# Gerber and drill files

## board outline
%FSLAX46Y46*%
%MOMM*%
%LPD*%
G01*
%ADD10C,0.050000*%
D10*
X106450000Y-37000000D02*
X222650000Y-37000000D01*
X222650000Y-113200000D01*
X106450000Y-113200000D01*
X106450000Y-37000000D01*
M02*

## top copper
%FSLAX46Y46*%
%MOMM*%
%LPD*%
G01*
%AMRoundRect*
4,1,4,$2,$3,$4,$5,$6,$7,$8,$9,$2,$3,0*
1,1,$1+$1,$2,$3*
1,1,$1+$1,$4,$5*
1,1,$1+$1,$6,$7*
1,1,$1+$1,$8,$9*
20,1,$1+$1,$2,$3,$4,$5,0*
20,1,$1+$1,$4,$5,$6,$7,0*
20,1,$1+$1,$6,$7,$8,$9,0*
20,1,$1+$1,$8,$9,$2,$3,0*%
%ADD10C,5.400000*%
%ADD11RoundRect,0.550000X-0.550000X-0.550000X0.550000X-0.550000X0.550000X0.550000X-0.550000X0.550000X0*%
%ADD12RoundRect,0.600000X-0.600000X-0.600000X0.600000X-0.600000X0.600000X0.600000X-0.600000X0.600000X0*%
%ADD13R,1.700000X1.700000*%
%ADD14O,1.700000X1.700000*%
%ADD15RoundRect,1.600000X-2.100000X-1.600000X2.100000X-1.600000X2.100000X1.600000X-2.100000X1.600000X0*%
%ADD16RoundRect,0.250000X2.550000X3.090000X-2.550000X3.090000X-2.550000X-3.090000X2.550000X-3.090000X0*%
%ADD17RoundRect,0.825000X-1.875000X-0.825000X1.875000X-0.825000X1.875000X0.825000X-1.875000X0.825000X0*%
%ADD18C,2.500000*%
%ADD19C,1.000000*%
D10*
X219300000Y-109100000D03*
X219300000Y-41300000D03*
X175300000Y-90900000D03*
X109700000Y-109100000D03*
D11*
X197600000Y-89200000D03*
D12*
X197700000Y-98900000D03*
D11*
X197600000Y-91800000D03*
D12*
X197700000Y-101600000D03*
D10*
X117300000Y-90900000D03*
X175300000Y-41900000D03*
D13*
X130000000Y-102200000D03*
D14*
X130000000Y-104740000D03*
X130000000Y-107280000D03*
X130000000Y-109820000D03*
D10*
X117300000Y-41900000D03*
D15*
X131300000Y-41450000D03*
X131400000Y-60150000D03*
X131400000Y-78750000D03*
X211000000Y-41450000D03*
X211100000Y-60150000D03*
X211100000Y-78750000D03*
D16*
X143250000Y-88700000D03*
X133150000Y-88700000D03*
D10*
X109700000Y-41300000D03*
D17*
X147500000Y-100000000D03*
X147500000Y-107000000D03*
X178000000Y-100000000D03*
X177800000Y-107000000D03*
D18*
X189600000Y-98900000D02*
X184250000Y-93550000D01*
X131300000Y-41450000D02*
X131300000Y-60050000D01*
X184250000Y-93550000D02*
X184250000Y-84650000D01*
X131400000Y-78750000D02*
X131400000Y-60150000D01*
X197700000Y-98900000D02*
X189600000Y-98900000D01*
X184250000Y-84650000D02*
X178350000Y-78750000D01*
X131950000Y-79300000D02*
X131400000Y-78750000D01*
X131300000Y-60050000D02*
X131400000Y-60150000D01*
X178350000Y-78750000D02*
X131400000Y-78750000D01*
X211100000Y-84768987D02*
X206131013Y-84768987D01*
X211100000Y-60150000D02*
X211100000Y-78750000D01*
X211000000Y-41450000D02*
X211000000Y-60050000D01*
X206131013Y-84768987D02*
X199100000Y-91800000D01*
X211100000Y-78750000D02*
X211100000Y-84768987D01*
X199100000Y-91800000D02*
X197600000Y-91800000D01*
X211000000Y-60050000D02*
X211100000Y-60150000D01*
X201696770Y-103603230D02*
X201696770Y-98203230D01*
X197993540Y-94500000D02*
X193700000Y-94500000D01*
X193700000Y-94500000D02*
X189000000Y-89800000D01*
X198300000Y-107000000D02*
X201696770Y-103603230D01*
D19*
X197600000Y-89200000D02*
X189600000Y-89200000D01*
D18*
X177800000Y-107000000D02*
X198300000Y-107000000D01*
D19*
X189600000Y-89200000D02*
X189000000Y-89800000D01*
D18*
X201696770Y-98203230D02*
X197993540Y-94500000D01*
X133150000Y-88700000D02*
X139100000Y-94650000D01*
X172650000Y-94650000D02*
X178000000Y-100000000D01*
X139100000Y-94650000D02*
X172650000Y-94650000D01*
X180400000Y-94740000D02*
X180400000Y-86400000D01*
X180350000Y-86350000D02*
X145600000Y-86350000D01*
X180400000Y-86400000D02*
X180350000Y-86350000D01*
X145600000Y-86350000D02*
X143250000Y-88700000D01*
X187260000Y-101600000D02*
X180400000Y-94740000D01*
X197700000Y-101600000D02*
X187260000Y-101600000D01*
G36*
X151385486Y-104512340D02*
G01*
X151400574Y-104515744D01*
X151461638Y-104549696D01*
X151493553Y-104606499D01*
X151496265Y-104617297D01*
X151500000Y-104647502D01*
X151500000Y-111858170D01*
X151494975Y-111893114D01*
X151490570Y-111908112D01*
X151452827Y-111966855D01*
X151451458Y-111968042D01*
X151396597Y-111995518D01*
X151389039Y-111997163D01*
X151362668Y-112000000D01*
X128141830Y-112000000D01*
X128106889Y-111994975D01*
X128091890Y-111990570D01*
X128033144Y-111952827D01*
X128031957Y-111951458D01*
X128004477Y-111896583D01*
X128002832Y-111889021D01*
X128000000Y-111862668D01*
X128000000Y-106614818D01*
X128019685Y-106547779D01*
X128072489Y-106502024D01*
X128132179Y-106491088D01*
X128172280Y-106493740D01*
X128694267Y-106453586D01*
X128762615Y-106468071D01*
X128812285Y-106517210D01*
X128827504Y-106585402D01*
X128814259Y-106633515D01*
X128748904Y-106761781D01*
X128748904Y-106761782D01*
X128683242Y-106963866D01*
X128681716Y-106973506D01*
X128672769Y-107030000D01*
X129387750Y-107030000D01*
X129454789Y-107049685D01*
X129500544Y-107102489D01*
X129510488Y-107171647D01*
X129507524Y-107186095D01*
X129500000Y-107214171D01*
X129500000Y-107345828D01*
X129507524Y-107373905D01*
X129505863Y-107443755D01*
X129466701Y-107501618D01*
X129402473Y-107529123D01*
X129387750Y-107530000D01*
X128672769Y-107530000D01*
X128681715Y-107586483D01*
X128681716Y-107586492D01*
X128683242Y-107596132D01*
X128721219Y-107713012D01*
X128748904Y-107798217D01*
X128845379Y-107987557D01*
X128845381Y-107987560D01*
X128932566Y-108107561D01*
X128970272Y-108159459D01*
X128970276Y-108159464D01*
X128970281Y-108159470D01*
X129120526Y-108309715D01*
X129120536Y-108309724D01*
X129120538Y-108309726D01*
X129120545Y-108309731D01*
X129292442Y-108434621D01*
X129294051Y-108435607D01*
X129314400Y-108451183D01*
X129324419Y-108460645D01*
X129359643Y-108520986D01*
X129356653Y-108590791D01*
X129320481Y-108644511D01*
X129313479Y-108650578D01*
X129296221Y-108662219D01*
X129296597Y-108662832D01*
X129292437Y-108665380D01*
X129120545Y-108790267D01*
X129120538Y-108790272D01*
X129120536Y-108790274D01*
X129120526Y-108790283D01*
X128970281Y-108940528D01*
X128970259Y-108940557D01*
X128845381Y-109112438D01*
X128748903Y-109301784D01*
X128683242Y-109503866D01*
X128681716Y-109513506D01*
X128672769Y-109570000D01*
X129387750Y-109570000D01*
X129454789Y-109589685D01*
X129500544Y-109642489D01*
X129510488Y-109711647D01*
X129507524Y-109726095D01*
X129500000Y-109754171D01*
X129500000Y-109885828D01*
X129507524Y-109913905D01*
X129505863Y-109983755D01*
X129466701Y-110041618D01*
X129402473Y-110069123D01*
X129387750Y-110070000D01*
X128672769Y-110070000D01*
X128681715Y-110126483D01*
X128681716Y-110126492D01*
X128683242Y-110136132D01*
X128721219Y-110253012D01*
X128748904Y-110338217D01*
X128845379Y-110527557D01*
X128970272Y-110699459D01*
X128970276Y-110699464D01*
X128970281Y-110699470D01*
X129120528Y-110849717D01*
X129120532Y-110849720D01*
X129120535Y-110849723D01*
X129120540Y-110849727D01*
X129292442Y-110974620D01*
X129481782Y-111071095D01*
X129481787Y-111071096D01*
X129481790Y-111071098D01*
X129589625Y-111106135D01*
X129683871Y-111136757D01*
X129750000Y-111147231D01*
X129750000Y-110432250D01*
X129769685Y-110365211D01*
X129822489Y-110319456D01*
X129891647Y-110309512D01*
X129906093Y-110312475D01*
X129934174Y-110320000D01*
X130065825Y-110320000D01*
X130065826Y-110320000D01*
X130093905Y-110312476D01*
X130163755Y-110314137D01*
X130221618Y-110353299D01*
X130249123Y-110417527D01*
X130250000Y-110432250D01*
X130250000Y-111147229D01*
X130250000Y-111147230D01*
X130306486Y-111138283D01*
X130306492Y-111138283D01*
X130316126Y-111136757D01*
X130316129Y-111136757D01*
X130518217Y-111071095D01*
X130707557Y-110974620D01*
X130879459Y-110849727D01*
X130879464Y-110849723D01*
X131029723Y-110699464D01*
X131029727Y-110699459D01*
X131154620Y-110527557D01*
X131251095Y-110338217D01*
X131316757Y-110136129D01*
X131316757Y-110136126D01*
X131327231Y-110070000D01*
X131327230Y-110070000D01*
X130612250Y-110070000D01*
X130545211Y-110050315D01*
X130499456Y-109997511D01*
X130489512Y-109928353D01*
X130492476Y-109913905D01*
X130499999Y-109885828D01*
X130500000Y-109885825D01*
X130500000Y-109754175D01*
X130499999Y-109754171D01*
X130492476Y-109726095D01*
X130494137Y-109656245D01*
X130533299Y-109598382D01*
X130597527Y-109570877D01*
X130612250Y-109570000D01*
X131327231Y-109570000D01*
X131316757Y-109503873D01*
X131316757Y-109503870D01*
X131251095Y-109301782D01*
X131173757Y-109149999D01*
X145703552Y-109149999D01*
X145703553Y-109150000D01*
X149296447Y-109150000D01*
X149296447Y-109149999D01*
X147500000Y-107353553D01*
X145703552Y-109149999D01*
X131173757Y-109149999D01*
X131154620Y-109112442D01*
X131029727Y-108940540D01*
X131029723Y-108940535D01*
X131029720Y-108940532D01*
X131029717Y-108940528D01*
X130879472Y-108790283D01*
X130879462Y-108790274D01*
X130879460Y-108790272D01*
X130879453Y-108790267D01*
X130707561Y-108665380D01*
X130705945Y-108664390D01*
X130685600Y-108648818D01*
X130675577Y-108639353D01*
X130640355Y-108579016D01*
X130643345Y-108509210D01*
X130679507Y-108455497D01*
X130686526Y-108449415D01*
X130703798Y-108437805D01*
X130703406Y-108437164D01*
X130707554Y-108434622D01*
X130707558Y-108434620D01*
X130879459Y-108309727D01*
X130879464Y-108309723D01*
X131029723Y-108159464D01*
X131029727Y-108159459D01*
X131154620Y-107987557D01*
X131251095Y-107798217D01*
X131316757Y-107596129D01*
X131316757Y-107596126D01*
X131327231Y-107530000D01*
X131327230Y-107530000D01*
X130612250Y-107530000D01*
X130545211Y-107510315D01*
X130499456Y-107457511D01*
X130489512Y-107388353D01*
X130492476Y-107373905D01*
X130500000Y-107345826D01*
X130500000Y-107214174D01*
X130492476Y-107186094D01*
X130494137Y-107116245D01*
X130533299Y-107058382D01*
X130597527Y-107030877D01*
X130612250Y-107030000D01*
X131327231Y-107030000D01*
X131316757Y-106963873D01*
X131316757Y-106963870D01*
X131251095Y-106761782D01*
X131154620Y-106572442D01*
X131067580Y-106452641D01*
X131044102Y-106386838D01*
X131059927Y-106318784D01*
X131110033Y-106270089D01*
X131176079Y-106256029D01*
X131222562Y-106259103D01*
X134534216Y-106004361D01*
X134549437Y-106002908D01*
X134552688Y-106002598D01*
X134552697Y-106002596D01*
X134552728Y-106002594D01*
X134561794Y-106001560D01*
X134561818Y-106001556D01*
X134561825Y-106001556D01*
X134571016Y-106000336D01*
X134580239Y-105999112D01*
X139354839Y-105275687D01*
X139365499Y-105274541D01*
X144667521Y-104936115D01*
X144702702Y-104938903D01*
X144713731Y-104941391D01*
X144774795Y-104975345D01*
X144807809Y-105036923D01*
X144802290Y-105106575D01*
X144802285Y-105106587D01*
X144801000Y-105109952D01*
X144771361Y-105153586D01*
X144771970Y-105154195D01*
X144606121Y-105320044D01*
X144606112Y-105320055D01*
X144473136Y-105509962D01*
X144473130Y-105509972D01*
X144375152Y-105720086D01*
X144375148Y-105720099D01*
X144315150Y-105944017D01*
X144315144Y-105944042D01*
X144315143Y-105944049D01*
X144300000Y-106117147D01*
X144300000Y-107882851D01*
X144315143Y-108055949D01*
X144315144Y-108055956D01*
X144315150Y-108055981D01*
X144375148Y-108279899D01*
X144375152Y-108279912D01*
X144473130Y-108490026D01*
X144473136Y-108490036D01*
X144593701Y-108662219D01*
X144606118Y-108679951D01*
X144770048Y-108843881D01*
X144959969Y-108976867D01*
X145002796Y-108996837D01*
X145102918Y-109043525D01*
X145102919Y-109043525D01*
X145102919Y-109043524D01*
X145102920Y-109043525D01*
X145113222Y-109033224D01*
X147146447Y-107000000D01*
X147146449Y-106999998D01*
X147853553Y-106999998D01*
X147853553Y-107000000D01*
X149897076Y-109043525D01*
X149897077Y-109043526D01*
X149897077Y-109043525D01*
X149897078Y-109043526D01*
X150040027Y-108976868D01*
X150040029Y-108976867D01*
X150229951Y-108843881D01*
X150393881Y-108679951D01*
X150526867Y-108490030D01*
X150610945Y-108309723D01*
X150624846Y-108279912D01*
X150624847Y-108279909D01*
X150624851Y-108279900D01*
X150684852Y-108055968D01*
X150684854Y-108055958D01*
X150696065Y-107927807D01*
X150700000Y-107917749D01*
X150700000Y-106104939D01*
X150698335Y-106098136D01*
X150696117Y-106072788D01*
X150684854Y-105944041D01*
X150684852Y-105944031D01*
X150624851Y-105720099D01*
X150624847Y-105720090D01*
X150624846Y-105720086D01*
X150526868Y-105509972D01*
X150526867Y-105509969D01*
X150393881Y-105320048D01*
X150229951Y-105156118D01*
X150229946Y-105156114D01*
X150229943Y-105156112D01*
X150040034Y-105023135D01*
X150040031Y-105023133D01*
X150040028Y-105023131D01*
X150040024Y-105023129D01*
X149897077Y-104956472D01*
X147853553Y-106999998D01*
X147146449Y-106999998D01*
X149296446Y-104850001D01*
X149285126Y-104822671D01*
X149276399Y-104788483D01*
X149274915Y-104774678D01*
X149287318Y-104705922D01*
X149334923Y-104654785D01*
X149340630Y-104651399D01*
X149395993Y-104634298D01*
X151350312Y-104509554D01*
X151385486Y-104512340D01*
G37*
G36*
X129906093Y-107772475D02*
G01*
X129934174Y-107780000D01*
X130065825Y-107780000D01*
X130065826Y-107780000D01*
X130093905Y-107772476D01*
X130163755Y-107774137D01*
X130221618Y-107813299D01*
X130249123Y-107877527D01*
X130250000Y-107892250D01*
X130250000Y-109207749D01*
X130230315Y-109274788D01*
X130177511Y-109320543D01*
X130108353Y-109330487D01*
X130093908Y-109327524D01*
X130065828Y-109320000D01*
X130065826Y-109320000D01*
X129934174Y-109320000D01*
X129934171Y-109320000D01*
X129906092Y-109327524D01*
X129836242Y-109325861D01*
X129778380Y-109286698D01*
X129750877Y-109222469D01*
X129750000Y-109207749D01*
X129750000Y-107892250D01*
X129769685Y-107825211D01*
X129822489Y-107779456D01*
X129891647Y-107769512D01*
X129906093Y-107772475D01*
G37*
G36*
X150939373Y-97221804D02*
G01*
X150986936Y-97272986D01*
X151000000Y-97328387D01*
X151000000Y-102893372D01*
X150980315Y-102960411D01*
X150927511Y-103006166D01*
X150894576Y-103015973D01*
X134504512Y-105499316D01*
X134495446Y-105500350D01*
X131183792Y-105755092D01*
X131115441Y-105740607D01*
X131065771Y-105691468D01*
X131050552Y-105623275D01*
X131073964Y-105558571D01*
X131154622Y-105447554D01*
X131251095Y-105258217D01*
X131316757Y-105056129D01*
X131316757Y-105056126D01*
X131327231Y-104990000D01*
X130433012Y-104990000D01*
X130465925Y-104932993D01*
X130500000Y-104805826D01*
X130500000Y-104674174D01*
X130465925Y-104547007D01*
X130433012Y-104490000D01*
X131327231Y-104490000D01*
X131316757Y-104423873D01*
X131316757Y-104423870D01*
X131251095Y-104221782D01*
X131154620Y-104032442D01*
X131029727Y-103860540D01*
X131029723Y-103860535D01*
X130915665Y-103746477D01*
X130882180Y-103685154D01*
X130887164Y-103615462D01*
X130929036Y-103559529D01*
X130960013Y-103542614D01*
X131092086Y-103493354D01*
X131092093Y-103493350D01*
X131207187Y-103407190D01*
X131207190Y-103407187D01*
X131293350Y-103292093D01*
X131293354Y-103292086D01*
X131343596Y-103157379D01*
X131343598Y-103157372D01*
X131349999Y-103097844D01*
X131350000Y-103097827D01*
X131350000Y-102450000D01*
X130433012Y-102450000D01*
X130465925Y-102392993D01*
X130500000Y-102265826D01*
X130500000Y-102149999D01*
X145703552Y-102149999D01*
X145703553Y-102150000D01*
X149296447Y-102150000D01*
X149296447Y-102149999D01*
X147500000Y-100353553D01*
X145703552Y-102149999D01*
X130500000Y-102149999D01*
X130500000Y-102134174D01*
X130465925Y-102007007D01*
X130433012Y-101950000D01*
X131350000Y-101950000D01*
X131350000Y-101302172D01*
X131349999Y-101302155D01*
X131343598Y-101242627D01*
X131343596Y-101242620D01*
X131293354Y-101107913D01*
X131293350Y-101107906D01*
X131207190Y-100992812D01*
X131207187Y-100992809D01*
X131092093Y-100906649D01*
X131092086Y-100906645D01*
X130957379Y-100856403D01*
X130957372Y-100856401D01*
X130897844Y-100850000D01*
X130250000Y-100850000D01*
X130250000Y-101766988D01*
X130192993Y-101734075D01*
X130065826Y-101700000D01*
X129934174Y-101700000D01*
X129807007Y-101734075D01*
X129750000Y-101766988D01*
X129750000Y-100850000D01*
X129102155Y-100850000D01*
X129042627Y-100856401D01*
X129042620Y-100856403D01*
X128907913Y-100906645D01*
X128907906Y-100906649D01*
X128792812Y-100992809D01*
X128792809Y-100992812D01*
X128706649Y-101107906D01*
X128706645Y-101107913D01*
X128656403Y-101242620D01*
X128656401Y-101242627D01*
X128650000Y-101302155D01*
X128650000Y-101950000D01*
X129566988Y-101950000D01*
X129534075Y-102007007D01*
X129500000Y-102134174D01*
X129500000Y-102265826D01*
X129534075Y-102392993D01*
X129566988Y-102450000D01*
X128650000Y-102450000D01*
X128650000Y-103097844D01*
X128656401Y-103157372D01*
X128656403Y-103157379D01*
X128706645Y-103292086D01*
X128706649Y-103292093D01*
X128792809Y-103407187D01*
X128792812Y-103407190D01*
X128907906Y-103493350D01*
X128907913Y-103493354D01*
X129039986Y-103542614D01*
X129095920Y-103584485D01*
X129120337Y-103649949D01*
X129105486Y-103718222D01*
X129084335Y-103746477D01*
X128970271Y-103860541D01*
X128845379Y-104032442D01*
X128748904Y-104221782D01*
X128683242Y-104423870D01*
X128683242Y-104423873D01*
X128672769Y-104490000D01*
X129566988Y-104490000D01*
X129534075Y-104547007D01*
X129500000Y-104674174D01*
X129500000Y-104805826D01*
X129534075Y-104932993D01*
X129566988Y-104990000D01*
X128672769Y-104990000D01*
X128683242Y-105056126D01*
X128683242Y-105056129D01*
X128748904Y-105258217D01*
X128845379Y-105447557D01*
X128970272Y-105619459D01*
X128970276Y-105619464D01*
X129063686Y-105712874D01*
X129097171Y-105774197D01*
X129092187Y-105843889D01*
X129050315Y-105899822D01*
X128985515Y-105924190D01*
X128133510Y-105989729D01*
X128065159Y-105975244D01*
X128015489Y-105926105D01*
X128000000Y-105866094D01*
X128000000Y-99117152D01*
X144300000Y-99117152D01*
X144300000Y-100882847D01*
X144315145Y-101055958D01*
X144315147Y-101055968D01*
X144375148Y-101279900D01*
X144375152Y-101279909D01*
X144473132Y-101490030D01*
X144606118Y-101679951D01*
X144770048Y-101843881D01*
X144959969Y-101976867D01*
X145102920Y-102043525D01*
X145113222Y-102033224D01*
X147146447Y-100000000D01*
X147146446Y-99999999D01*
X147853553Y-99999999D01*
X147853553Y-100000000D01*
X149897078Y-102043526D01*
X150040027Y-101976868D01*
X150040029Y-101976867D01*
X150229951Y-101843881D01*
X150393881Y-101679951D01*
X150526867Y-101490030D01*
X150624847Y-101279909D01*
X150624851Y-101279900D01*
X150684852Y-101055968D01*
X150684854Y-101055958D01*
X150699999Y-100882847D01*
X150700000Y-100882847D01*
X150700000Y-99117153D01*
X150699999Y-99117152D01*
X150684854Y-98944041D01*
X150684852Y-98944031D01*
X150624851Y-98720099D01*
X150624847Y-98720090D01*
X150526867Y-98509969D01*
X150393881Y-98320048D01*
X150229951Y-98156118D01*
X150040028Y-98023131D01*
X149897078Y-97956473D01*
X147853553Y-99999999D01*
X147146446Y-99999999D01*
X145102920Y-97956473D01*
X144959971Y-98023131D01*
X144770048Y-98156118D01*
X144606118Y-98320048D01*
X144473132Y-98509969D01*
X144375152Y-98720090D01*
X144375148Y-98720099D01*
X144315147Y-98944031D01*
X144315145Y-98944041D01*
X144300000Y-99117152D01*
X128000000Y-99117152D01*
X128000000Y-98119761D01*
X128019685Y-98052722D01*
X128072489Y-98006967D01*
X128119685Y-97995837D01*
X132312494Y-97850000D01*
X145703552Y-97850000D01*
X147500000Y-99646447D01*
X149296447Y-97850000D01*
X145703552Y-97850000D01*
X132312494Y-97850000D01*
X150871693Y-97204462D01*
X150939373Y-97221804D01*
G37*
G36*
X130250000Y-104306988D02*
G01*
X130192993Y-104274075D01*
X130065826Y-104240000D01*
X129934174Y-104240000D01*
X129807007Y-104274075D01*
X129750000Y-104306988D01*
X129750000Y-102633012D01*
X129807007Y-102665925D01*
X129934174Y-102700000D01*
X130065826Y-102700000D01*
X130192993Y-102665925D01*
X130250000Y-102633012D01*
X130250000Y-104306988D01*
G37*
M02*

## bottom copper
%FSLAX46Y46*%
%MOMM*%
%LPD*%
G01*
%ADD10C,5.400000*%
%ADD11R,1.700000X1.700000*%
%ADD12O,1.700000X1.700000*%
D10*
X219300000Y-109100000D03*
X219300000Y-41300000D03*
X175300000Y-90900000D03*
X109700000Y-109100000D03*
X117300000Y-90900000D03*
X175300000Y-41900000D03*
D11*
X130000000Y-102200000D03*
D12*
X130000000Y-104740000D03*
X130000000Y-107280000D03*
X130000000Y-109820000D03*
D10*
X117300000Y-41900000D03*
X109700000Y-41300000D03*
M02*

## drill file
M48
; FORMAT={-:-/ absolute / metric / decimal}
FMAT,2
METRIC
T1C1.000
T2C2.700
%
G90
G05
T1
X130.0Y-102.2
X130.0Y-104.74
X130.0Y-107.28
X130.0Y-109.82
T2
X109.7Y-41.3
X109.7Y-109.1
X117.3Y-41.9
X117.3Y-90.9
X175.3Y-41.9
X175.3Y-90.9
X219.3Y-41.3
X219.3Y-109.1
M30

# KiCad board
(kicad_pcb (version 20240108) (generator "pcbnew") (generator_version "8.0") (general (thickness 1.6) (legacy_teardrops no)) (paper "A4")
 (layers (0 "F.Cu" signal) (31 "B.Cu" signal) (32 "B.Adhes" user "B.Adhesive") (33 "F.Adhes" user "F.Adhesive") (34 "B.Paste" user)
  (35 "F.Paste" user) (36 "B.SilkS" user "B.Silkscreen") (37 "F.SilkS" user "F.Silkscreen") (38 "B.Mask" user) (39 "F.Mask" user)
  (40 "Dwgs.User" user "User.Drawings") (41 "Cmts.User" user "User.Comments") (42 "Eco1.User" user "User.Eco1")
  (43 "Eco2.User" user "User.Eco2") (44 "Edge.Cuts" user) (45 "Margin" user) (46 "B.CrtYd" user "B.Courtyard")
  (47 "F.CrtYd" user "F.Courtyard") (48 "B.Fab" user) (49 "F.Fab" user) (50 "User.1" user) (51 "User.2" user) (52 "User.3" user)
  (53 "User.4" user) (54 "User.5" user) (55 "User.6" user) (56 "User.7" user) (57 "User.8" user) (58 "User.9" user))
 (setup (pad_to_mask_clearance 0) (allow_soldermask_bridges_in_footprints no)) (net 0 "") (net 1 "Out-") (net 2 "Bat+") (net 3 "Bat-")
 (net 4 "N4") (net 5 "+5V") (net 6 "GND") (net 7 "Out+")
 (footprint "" (layer "F.Cu") (at 219.3 109.1)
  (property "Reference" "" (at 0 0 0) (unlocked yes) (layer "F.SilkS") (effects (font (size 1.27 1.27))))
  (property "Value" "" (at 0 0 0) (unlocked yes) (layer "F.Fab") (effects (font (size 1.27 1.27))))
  (pad "1" thru_hole circle (at 0 0) (size 5.4 5.4) (drill 2.7) (layers "*.Cu" "*.Mask") (remove_unused_layers no)))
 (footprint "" (layer "F.Cu") (at 219.3 41.3)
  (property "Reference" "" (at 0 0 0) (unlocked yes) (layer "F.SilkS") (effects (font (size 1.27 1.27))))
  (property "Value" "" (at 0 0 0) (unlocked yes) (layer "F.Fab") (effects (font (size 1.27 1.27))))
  (pad "1" thru_hole circle (at 0 0) (size 5.4 5.4) (drill 2.7) (layers "*.Cu" "*.Mask") (remove_unused_layers no)))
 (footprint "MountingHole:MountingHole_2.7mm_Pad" (layer "F.Cu") (at 175.3 90.9)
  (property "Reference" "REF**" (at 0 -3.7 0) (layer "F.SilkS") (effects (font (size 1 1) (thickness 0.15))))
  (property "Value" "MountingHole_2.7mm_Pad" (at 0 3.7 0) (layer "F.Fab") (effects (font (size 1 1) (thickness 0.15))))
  (pad "1" thru_hole circle (at 0 0) (size 5.4 5.4) (drill 2.7) (layers "*.Cu" "*.Mask") (remove_unused_layers no)))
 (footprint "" (layer "F.Cu") (at 109.7 109.1)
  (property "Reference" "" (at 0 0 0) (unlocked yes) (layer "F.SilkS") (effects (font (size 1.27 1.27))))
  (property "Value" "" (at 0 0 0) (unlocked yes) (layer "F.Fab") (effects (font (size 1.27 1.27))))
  (pad "1" thru_hole circle (at 0 0) (size 5.4 5.4) (drill 2.7) (layers "*.Cu" "*.Mask") (remove_unused_layers no)))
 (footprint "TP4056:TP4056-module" (layer "F.Cu") (at 208.3 96)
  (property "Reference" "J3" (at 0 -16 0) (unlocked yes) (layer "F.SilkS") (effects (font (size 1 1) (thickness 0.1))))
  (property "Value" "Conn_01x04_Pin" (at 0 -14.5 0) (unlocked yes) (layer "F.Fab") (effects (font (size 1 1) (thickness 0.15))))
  (pad "1" smd roundrect (at -10.7 -6.8) (size 2.2 2.2) (layers "F.Cu" "F.Paste" "F.Mask") (roundrect_rratio 0.25) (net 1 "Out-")
   (thermal_bridge_angle 45))
  (pad "2" smd roundrect (at -10.6 2.9) (size 2.4 2.4) (layers "F.Cu" "F.Paste" "F.Mask") (roundrect_rratio 0.25) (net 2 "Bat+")
   (thermal_bridge_angle 45))
  (pad "3" smd roundrect (at -10.7 -4.2) (size 2.2 2.2) (layers "F.Cu" "F.Paste" "F.Mask") (roundrect_rratio 0.25) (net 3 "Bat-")
   (thermal_bridge_angle 45))
  (pad "4" smd roundrect (at -10.6 5.6) (size 2.4 2.4) (layers "F.Cu" "F.Paste" "F.Mask") (roundrect_rratio 0.25) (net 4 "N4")
   (thermal_bridge_angle 45)))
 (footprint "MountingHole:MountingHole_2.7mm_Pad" (layer "F.Cu") (at 117.3 90.9)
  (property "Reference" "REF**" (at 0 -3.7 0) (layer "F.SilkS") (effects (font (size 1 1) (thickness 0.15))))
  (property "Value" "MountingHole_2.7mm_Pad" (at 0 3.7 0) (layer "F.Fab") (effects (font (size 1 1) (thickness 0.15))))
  (pad "1" thru_hole circle (at 0 0) (size 5.4 5.4) (drill 2.7) (layers "*.Cu" "*.Mask") (remove_unused_layers no)))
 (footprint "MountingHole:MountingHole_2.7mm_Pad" (layer "F.Cu") (at 175.3 41.9)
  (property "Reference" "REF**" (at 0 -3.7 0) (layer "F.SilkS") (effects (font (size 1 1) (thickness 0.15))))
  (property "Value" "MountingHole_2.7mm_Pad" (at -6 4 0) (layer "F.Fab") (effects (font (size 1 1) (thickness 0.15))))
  (pad "1" thru_hole circle (at 0 0) (size 5.4 5.4) (drill 2.7) (layers "*.Cu" "*.Mask") (remove_unused_layers no)))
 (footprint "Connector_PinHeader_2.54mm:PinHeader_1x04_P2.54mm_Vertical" (layer "F.Cu") (at 130 102.2)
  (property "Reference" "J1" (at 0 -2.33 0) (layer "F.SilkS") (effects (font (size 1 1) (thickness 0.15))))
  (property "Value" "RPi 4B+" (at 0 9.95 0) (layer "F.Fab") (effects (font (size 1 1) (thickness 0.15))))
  (pad "1" thru_hole rect (at 0 0) (size 1.7 1.7) (drill 1) (layers "*.Cu" "*.Mask") (remove_unused_layers no) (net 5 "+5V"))
  (pad "2" thru_hole oval (at 0 2.54) (size 1.7 1.7) (drill 1) (layers "*.Cu" "*.Mask") (remove_unused_layers no) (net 5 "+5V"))
  (pad "3" thru_hole oval (at 0 5.08) (size 1.7 1.7) (drill 1) (layers "*.Cu" "*.Mask") (remove_unused_layers no) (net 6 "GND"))
  (pad "4" thru_hole oval (at 0 7.62) (size 1.7 1.7) (drill 1) (layers "*.Cu" "*.Mask") (remove_unused_layers no) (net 6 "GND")))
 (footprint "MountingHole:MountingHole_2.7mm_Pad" (layer "F.Cu") (at 117.3 41.9)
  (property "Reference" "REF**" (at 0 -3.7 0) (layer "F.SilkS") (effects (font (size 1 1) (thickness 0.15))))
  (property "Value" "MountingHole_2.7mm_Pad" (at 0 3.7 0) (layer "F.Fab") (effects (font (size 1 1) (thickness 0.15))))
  (pad "1" thru_hole circle (at 0 0) (size 5.4 5.4) (drill 2.7) (layers "*.Cu" "*.Mask") (remove_unused_layers no)))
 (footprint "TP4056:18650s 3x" (layer "F.Cu") (at 127.6 38.35)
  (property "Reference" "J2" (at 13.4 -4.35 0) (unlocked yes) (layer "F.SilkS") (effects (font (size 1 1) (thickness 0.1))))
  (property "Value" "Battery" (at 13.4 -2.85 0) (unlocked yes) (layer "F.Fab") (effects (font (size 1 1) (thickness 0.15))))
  (pad "1" smd roundrect (at 3.7 3.1) (size 7.4 6.4) (layers "F.Cu" "F.Paste" "F.Mask") (roundrect_rratio 0.25) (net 2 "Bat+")
   (thermal_bridge_angle 45))
  (pad "1" smd roundrect (at 3.8 21.8) (size 7.4 6.4) (layers "F.Cu" "F.Paste" "F.Mask") (roundrect_rratio 0.25) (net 2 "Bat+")
   (thermal_bridge_angle 45))
  (pad "1" smd roundrect (at 3.8 40.4) (size 7.4 6.4) (layers "F.Cu" "F.Paste" "F.Mask") (roundrect_rratio 0.25) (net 2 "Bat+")
   (thermal_bridge_angle 45))
  (pad "2" smd roundrect (at 83.4 3.1) (size 7.4 6.4) (layers "F.Cu" "F.Paste" "F.Mask") (roundrect_rratio 0.25) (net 3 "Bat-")
   (thermal_bridge_angle 45))
  (pad "2" smd roundrect (at 83.5 21.8) (size 7.4 6.4) (layers "F.Cu" "F.Paste" "F.Mask") (roundrect_rratio 0.25) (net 3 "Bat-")
   (thermal_bridge_angle 45))
  (pad "2" smd roundrect (at 83.5 40.4) (size 7.4 6.4) (layers "F.Cu" "F.Paste" "F.Mask") (roundrect_rratio 0.25) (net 3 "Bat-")
   (thermal_bridge_angle 45)))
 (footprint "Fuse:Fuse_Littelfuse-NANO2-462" (layer "F.Cu") (at 138.2 88.7 180)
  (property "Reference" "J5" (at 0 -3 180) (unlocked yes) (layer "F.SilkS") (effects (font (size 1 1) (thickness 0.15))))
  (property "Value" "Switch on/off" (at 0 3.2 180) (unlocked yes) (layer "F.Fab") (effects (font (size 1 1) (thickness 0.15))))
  (pad "1" smd roundrect (at -5.05 0 180) (size 5.6 6.68) (layers "F.Cu" "F.Paste" "F.Mask") (roundrect_rratio 0.04464285714) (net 4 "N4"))
  (pad "2" smd roundrect (at 5.05 0 180) (size 5.6 6.68) (layers "F.Cu" "F.Paste" "F.Mask") (roundrect_rratio 0.04464285714) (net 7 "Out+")))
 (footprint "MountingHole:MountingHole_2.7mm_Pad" (layer "F.Cu") (at 109.7 41.3)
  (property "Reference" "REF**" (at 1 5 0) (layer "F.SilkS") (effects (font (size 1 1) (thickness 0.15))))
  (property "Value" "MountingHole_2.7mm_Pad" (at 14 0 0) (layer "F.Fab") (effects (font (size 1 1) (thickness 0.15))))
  (pad "1" thru_hole circle (at 0 0) (size 5.4 5.4) (drill 2.7) (layers "*.Cu" "*.Mask") (remove_unused_layers no)))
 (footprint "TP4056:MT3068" (layer "F.Cu") (at 162.7 103.45)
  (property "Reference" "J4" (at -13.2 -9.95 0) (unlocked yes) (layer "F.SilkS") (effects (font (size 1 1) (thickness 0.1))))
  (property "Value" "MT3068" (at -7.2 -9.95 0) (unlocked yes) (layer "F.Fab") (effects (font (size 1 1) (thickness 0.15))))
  (pad "1" smd roundrect (at -15.2 -3.45) (size 5.4 3.3) (layers "F.Cu" "F.Paste" "F.Mask") (roundrect_rratio 0.25) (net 5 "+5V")
   (thermal_bridge_angle 45))
  (pad "2" smd roundrect (at -15.2 3.55) (size 5.4 3.3) (layers "F.Cu" "F.Paste" "F.Mask") (roundrect_rratio 0.25) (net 6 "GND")
   (thermal_bridge_angle 45))
  (pad "3" smd roundrect (at 15.3 -3.45) (size 5.4 3.3) (layers "F.Cu" "F.Paste" "F.Mask") (roundrect_rratio 0.25) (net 7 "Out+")
   (thermal_bridge_angle 45))
  (pad "4" smd roundrect (at 15.1 3.55) (size 5.4 3.3) (layers "F.Cu" "F.Paste" "F.Mask") (roundrect_rratio 0.25) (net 1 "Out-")
   (thermal_bridge_angle 45)))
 (gr_rect (start 106.45 37) (end 222.65 113.2) (stroke (width 0.05) (type default)) (fill none) (layer "Edge.Cuts"))
 (segment (start 189.6 98.9) (end 184.25 93.55) (width 2.5) (layer "F.Cu") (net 2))
 (segment (start 131.3 41.45) (end 131.3 60.05) (width 2.5) (layer "F.Cu") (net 2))
 (segment (start 184.25 93.55) (end 184.25 84.65) (width 2.5) (layer "F.Cu") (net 2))
 (segment (start 131.4 78.75) (end 131.4 60.15) (width 2.5) (layer "F.Cu") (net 2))
 (segment (start 197.7 98.9) (end 189.6 98.9) (width 2.5) (layer "F.Cu") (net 2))
 (segment (start 184.25 84.65) (end 178.35 78.75) (width 2.5) (layer "F.Cu") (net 2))
 (segment (start 131.95 79.3) (end 131.4 78.75) (width 2.5) (layer "F.Cu") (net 2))
 (segment (start 131.3 60.05) (end 131.4 60.15) (width 2.5) (layer "F.Cu") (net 2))
 (segment (start 178.35 78.75) (end 131.4 78.75) (width 2.5) (layer "F.Cu") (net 2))
 (segment (start 211.1 84.768987) (end 206.131013 84.768987) (width 2.5) (layer "F.Cu") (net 3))
 (segment (start 211.1 60.15) (end 211.1 78.75) (width 2.5) (layer "F.Cu") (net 3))
 (segment (start 211 41.45) (end 211 60.05) (width 2.5) (layer "F.Cu") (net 3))
 (segment (start 206.131013 84.768987) (end 199.1 91.8) (width 2.5) (layer "F.Cu") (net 3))
 (segment (start 211.1 78.75) (end 211.1 84.768987) (width 2.5) (layer "F.Cu") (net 3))
 (segment (start 199.1 91.8) (end 197.6 91.8) (width 2.5) (layer "F.Cu") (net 3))
 (segment (start 211 60.05) (end 211.1 60.15) (width 2.5) (layer "F.Cu") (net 3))
 (segment (start 201.69677 103.60323) (end 201.69677 98.20323) (width 2.5) (layer "F.Cu") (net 1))
 (segment (start 197.99354 94.5) (end 193.7 94.5) (width 2.5) (layer "F.Cu") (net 1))
 (segment (start 193.7 94.5) (end 189 89.8) (width 2.5) (layer "F.Cu") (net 1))
 (segment (start 198.3 107) (end 201.69677 103.60323) (width 2.5) (layer "F.Cu") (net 1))
 (segment (start 197.6 89.2) (end 189.6 89.2) (width 1) (layer "F.Cu") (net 1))
 (segment (start 177.8 107) (end 198.3 107) (width 2.5) (layer "F.Cu") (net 1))
 (segment (start 189.6 89.2) (end 189 89.8) (width 1) (layer "F.Cu") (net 1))
 (segment (start 201.69677 98.20323) (end 197.99354 94.5) (width 2.5) (layer "F.Cu") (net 1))
 (segment (start 133.15 88.7) (end 139.1 94.65) (width 2.5) (layer "F.Cu") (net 7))
 (segment (start 172.65 94.65) (end 178 100) (width 2.5) (layer "F.Cu") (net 7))
 (segment (start 139.1 94.65) (end 172.65 94.65) (width 2.5) (layer "F.Cu") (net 7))
 (segment (start 180.4 94.74) (end 180.4 86.4) (width 2.5) (layer "F.Cu") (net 4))
 (segment (start 180.35 86.35) (end 145.6 86.35) (width 2.5) (layer "F.Cu") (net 4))
 (segment (start 180.4 86.4) (end 180.35 86.35) (width 2.5) (layer "F.Cu") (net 4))
 (segment (start 145.6 86.35) (end 143.25 88.7) (width 2.5) (layer "F.Cu") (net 4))
 (segment (start 187.26 101.6) (end 180.4 94.74) (width 2.5) (layer "F.Cu") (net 4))
 (segment (start 197.7 101.6) (end 187.26 101.6) (width 2.5) (layer "F.Cu") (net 4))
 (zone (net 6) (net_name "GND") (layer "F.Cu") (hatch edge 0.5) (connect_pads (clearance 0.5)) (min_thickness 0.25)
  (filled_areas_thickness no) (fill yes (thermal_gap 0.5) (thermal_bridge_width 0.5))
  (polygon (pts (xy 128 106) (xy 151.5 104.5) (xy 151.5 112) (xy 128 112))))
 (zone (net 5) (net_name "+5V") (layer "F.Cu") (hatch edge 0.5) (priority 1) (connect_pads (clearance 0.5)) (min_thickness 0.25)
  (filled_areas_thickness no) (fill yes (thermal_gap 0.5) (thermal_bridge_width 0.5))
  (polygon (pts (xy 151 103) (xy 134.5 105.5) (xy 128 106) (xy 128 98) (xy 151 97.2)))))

